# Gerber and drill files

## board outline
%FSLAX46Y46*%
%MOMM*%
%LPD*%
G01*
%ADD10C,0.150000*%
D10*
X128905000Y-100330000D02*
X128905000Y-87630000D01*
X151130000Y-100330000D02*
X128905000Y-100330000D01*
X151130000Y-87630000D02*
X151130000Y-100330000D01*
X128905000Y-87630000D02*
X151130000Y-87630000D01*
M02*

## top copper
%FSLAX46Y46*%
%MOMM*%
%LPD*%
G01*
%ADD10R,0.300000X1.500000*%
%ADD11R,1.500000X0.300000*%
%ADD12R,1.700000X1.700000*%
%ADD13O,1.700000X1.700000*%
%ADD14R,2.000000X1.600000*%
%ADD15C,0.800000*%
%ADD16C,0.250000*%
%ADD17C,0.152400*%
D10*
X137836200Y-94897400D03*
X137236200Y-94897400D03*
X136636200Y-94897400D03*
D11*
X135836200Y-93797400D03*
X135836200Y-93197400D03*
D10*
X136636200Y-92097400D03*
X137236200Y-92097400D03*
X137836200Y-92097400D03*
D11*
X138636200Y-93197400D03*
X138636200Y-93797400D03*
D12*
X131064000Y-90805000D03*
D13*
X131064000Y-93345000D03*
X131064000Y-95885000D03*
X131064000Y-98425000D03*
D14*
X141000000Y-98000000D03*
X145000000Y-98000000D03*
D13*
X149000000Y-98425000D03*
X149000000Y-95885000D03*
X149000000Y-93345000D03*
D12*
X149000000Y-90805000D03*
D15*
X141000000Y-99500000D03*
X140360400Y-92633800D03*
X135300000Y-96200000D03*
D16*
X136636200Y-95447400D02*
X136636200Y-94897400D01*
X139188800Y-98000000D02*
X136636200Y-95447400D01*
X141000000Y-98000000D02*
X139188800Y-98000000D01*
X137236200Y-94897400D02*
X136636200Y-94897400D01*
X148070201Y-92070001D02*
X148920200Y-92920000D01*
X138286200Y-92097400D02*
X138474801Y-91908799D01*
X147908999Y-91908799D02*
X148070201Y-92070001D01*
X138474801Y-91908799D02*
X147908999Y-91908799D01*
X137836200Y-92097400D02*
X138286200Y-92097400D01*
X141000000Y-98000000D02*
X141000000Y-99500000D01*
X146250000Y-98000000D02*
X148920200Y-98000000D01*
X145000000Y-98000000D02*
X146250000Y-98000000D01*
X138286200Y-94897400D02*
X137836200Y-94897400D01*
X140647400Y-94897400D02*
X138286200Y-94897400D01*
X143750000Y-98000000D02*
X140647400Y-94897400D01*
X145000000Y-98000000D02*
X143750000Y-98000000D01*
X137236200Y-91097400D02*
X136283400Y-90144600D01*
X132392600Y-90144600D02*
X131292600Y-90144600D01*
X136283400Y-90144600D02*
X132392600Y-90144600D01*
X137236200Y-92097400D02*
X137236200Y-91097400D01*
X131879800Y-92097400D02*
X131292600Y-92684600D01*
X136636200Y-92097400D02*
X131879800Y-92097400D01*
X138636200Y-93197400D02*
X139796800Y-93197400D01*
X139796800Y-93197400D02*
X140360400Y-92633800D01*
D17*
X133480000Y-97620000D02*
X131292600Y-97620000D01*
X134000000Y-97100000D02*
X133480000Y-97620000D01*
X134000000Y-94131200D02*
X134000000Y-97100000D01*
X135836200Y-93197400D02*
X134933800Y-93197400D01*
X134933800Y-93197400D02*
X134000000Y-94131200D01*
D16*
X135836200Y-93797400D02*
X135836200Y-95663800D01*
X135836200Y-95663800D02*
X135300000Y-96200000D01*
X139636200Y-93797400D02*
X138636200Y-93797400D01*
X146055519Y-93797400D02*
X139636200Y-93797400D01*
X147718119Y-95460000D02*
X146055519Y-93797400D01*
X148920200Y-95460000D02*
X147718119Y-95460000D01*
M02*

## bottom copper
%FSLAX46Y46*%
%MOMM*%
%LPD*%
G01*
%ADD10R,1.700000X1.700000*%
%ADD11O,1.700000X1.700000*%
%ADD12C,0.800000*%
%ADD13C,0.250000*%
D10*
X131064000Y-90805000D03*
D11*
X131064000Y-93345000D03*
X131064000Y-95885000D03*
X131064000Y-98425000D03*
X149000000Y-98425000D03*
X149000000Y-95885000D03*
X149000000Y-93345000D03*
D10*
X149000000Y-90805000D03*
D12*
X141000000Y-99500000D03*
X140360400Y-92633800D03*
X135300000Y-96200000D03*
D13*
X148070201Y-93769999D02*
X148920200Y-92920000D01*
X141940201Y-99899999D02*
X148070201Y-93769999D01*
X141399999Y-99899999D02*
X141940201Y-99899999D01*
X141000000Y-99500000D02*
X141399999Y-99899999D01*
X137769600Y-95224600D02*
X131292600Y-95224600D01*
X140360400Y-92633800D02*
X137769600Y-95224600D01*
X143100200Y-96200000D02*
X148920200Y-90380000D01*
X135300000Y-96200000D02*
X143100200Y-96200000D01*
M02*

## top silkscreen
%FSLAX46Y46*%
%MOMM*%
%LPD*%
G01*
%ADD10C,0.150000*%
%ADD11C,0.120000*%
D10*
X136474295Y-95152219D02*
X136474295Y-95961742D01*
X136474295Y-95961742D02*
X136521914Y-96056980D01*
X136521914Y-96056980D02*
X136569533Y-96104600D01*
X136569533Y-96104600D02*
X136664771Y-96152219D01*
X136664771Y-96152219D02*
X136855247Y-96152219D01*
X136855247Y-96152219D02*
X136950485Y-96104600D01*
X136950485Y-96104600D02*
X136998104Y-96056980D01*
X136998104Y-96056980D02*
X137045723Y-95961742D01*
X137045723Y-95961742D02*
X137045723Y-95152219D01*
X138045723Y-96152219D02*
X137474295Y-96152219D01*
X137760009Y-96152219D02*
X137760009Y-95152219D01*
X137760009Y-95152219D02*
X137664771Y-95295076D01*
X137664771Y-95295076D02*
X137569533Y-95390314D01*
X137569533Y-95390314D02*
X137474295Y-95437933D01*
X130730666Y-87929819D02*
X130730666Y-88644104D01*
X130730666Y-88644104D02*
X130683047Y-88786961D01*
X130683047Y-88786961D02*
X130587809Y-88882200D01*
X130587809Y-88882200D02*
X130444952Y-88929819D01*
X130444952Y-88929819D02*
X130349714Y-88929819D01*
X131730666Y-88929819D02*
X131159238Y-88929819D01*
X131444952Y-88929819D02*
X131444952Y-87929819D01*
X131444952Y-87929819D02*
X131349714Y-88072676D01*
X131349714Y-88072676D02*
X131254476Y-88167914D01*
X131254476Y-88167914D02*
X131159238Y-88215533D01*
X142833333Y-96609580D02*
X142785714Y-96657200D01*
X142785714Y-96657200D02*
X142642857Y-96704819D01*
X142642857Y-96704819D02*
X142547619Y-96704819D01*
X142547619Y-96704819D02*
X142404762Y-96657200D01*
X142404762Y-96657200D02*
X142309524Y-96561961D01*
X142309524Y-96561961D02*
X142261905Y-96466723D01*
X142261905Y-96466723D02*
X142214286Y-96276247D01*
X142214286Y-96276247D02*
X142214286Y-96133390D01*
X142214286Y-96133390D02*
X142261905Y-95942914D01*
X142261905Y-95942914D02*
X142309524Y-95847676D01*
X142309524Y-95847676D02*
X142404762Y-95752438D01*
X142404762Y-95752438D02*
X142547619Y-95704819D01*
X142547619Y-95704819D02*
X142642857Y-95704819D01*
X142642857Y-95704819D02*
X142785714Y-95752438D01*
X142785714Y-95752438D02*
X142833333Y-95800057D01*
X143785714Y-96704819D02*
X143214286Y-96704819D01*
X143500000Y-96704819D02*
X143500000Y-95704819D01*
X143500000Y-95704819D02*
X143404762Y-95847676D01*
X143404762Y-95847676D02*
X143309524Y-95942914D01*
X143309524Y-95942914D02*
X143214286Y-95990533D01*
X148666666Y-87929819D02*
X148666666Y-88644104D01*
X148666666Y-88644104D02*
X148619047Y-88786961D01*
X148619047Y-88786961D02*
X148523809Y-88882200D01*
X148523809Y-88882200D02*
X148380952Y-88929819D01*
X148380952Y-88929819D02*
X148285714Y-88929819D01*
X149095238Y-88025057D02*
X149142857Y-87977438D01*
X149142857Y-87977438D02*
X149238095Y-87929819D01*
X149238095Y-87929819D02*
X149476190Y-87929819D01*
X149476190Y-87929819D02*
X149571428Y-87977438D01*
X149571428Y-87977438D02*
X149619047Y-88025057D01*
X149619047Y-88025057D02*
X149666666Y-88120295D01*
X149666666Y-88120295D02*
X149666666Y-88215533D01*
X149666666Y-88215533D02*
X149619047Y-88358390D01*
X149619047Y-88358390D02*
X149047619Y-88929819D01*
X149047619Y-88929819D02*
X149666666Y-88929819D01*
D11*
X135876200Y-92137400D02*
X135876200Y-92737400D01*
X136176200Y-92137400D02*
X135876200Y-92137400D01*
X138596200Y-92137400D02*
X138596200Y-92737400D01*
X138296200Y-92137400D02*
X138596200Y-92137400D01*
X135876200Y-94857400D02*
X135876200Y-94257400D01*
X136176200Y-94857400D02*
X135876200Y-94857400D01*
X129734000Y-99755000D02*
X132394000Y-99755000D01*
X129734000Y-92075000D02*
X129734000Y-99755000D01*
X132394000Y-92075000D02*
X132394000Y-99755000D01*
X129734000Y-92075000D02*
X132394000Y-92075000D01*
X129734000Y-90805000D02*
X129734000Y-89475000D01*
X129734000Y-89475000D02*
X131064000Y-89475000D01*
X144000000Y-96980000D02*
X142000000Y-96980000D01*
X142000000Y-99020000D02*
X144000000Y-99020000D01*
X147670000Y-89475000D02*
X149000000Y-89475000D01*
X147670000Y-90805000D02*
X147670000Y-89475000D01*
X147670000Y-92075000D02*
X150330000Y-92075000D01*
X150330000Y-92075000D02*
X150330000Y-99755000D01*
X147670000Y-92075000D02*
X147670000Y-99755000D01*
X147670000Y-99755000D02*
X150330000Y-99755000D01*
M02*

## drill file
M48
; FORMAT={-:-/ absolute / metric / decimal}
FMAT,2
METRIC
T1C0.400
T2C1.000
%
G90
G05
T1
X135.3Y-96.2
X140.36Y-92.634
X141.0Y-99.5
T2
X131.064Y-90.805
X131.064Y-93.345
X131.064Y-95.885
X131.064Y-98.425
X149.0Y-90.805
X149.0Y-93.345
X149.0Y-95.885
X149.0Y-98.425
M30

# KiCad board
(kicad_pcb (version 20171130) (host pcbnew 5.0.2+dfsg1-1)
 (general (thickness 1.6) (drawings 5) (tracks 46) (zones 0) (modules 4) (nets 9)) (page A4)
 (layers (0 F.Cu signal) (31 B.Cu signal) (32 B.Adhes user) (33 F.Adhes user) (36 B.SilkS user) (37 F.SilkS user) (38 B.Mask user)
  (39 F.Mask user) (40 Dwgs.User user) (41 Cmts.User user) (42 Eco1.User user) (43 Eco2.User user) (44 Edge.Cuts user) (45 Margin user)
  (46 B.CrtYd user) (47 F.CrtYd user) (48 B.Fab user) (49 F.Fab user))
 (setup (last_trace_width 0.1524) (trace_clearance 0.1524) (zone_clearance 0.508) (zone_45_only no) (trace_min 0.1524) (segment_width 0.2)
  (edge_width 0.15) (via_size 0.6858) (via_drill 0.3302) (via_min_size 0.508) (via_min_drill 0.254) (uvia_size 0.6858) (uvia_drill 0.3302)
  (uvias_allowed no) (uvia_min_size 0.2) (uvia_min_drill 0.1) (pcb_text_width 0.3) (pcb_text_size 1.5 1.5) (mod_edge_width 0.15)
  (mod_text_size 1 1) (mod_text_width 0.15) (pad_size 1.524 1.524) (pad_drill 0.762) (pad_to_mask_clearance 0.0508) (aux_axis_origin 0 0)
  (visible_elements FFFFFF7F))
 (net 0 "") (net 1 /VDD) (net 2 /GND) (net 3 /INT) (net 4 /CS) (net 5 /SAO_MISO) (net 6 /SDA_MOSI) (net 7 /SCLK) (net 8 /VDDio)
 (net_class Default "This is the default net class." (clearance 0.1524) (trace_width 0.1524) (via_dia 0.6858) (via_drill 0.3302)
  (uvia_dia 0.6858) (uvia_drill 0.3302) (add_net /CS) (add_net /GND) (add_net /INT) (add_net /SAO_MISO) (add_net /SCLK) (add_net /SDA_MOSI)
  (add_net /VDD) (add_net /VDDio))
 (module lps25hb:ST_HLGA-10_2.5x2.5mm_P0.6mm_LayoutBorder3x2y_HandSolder (layer F.Cu) (at 137.2362 93.4974 180)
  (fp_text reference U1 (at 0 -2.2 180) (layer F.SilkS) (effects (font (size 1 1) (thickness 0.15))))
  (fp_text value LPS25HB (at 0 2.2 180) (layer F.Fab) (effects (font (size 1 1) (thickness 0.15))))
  (fp_line (start 1.36 1.36) (end 1.36 0.76) (layer F.SilkS) (width 0.12))
  (fp_line (start 1.06 1.36) (end 1.36 1.36) (layer F.SilkS) (width 0.12))
  (fp_line (start -1.36 1.36) (end -1.36 0.76) (layer F.SilkS) (width 0.12))
  (fp_line (start -1.06 1.36) (end -1.36 1.36) (layer F.SilkS) (width 0.12))
  (fp_line (start 1.36 -1.36) (end 1.36 -0.76) (layer F.SilkS) (width 0.12))
  (fp_line (start 1.06 -1.36) (end 1.36 -1.36) (layer F.SilkS) (width 0.12))
  (pad 10 smd rect (at -0.6 -1.4 180) (size 0.3 1.5) (layers F.Cu F.Paste F.Mask) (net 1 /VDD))
  (pad 9 smd rect (at 0 -1.4 180) (size 0.3 1.5) (layers F.Cu F.Paste F.Mask) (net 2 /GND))
  (pad 8 smd rect (at 0.6 -1.4 180) (size 0.3 1.5) (layers F.Cu F.Paste F.Mask) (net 2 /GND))
  (pad 7 smd rect (at 1.4 -0.3 180) (size 1.5 0.3) (layers F.Cu F.Paste F.Mask) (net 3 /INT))
  (pad 6 smd rect (at 1.4 0.3 180) (size 1.5 0.3) (layers F.Cu F.Paste F.Mask) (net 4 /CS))
  (pad 5 smd rect (at 0.6 1.4 180) (size 0.3 1.5) (layers F.Cu F.Paste F.Mask) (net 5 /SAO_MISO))
  (pad 4 smd rect (at 0 1.4 180) (size 0.3 1.5) (layers F.Cu F.Paste F.Mask) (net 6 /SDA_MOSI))
  (pad 3 smd rect (at -0.6 1.4 180) (size 0.3 1.5) (layers F.Cu F.Paste F.Mask) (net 2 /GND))
  (pad 2 smd rect (at -1.4 0.3 180) (size 1.5 0.3) (layers F.Cu F.Paste F.Mask) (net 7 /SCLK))
  (pad 1 smd rect (at -1.4 -0.3 180) (size 1.5 0.3) (layers F.Cu F.Paste F.Mask) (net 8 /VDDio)))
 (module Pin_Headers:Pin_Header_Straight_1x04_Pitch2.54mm (layer F.Cu) (at 131.064 90.805)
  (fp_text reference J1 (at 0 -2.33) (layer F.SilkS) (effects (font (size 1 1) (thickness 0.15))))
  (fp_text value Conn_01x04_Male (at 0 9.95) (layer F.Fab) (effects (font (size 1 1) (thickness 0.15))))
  (fp_line (start -1.33 8.95) (end 1.33 8.95) (layer F.SilkS) (width 0.12))
  (fp_line (start -1.33 1.27) (end -1.33 8.95) (layer F.SilkS) (width 0.12))
  (fp_line (start 1.33 1.27) (end 1.33 8.95) (layer F.SilkS) (width 0.12))
  (fp_line (start -1.33 1.27) (end 1.33 1.27) (layer F.SilkS) (width 0.12))
  (fp_line (start -1.33 0) (end -1.33 -1.33) (layer F.SilkS) (width 0.12))
  (fp_line (start -1.33 -1.33) (end 0 -1.33) (layer F.SilkS) (width 0.12))
  (pad 1 thru_hole rect (at 0 0) (size 1.7 1.7) (drill 1) (layers *.Cu *.Mask) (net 6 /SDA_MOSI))
  (pad 2 thru_hole oval (at 0 2.54) (size 1.7 1.7) (drill 1) (layers *.Cu *.Mask) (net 5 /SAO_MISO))
  (pad 3 thru_hole oval (at 0 5.08) (size 1.7 1.7) (drill 1) (layers *.Cu *.Mask) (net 7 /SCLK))
  (pad 4 thru_hole oval (at 0 7.62) (size 1.7 1.7) (drill 1) (layers *.Cu *.Mask) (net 4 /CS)))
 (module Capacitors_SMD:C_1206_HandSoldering (layer F.Cu) (at 143 98)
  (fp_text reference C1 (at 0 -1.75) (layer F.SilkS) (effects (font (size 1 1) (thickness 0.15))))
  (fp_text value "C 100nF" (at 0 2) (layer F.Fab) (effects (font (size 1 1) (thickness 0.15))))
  (fp_line (start 1 -1.02) (end -1 -1.02) (layer F.SilkS) (width 0.12))
  (fp_line (start -1 1.02) (end 1 1.02) (layer F.SilkS) (width 0.12))
  (pad 1 smd rect (at -2 0) (size 2 1.6) (layers F.Cu F.Paste F.Mask) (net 2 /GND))
  (pad 2 smd rect (at 2 0) (size 2 1.6) (layers F.Cu F.Paste F.Mask) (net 1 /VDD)))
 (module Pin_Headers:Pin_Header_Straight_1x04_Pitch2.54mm (layer F.Cu) (at 149 90.805)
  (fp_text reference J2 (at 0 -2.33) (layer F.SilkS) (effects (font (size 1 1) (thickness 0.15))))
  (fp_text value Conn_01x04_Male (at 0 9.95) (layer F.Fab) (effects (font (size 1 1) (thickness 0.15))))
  (fp_line (start -1.33 -1.33) (end 0 -1.33) (layer F.SilkS) (width 0.12))
  (fp_line (start -1.33 0) (end -1.33 -1.33) (layer F.SilkS) (width 0.12))
  (fp_line (start -1.33 1.27) (end 1.33 1.27) (layer F.SilkS) (width 0.12))
  (fp_line (start 1.33 1.27) (end 1.33 8.95) (layer F.SilkS) (width 0.12))
  (fp_line (start -1.33 1.27) (end -1.33 8.95) (layer F.SilkS) (width 0.12))
  (fp_line (start -1.33 8.95) (end 1.33 8.95) (layer F.SilkS) (width 0.12))
  (pad 4 thru_hole oval (at 0 7.62) (size 1.7 1.7) (drill 1) (layers *.Cu *.Mask) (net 1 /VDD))
  (pad 3 thru_hole oval (at 0 5.08) (size 1.7 1.7) (drill 1) (layers *.Cu *.Mask) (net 8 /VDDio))
  (pad 2 thru_hole oval (at 0 2.54) (size 1.7 1.7) (drill 1) (layers *.Cu *.Mask) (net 2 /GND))
  (pad 1 thru_hole rect (at 0 0) (size 1.7 1.7) (drill 1) (layers *.Cu *.Mask) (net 3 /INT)))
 (gr_line (start 128.905 100.33) (end 128.905 87.63) (layer Edge.Cuts) (width 0.15))
 (gr_line (start 151.13 100.33) (end 128.905 100.33) (layer Edge.Cuts) (width 0.15))
 (gr_line (start 151.13 87.63) (end 151.13 100.33) (layer Edge.Cuts) (width 0.15))
 (gr_line (start 128.905 87.63) (end 151.13 87.63) (layer Edge.Cuts) (width 0.15))
 (segment (start 136.6362 95.4474) (end 136.6362 94.8974) (width 0.25) (layer F.Cu) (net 2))
 (segment (start 139.1888 98) (end 136.6362 95.4474) (width 0.25) (layer F.Cu) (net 2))
 (segment (start 141 98) (end 139.1888 98) (width 0.25) (layer F.Cu) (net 2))
 (segment (start 137.2362 94.8974) (end 136.6362 94.8974) (width 0.25) (layer F.Cu) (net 2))
 (segment (start 148.070201 92.070001) (end 148.9202 92.92) (width 0.25) (layer F.Cu) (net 2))
 (segment (start 138.2862 92.0974) (end 138.474801 91.908799) (width 0.25) (layer F.Cu) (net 2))
 (segment (start 147.908999 91.908799) (end 148.070201 92.070001) (width 0.25) (layer F.Cu) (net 2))
 (segment (start 138.474801 91.908799) (end 147.908999 91.908799) (width 0.25) (layer F.Cu) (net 2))
 (segment (start 137.8362 92.0974) (end 138.2862 92.0974) (width 0.25) (layer F.Cu) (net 2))
 (via (at 141 99.5) (size 0.8) (drill 0.4) (layers F.Cu B.Cu) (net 2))
 (segment (start 141 98) (end 141 99.5) (width 0.25) (layer F.Cu) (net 2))
 (segment (start 148.070201 93.769999) (end 148.9202 92.92) (width 0.25) (layer B.Cu) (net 2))
 (segment (start 141.940201 99.899999) (end 148.070201 93.769999) (width 0.25) (layer B.Cu) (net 2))
 (segment (start 141.399999 99.899999) (end 141.940201 99.899999) (width 0.25) (layer B.Cu) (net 2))
 (segment (start 141 99.5) (end 141.399999 99.899999) (width 0.25) (layer B.Cu) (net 2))
 (segment (start 146.25 98) (end 148.9202 98) (width 0.25) (layer F.Cu) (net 1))
 (segment (start 145 98) (end 146.25 98) (width 0.25) (layer F.Cu) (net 1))
 (segment (start 138.2862 94.8974) (end 137.8362 94.8974) (width 0.25) (layer F.Cu) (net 1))
 (segment (start 140.6474 94.8974) (end 138.2862 94.8974) (width 0.25) (layer F.Cu) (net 1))
 (segment (start 143.75 98) (end 140.6474 94.8974) (width 0.25) (layer F.Cu) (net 1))
 (segment (start 145 98) (end 143.75 98) (width 0.25) (layer F.Cu) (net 1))
 (segment (start 137.2362 91.0974) (end 136.2834 90.1446) (width 0.25) (layer F.Cu) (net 6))
 (segment (start 132.3926 90.1446) (end 131.2926 90.1446) (width 0.25) (layer F.Cu) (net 6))
 (segment (start 136.2834 90.1446) (end 132.3926 90.1446) (width 0.25) (layer F.Cu) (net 6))
 (segment (start 137.2362 92.0974) (end 137.2362 91.0974) (width 0.25) (layer F.Cu) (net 6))
 (segment (start 131.8798 92.0974) (end 131.2926 92.6846) (width 0.25) (layer F.Cu) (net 5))
 (segment (start 136.6362 92.0974) (end 131.8798 92.0974) (width 0.25) (layer F.Cu) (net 5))
 (via (at 140.3604 92.6338) (size 0.8) (drill 0.4) (layers F.Cu B.Cu) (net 7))
 (segment (start 138.6362 93.1974) (end 139.7968 93.1974) (width 0.25) (layer F.Cu) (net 7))
 (segment (start 139.7968 93.1974) (end 140.3604 92.6338) (width 0.25) (layer F.Cu) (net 7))
 (segment (start 137.7696 95.2246) (end 131.2926 95.2246) (width 0.25) (layer B.Cu) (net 7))
 (segment (start 140.3604 92.6338) (end 137.7696 95.2246) (width 0.25) (layer B.Cu) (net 7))
 (segment (start 133.48 97.62) (end 131.2926 97.62) (width 0.1524) (layer F.Cu) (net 4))
 (segment (start 134 97.1) (end 133.48 97.62) (width 0.1524) (layer F.Cu) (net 4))
 (segment (start 134 94.1312) (end 134 97.1) (width 0.1524) (layer F.Cu) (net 4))
 (segment (start 135.8362 93.1974) (end 134.9338 93.1974) (width 0.1524) (layer F.Cu) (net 4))
 (segment (start 134.9338 93.1974) (end 134 94.1312) (width 0.1524) (layer F.Cu) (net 4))
 (via (at 135.3 96.2) (size 0.8) (drill 0.4) (layers F.Cu B.Cu) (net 3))
 (segment (start 135.8362 93.7974) (end 135.8362 95.6638) (width 0.25) (layer F.Cu) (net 3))
 (segment (start 135.8362 95.6638) (end 135.3 96.2) (width 0.25) (layer F.Cu) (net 3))
 (segment (start 143.1002 96.2) (end 148.9202 90.38) (width 0.25) (layer B.Cu) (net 3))
 (segment (start 135.3 96.2) (end 143.1002 96.2) (width 0.25) (layer B.Cu) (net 3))
 (segment (start 139.6362 93.7974) (end 138.6362 93.7974) (width 0.25) (layer F.Cu) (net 8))
 (segment (start 146.055519 93.7974) (end 139.6362 93.7974) (width 0.25) (layer F.Cu) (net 8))
 (segment (start 147.718119 95.46) (end 146.055519 93.7974) (width 0.25) (layer F.Cu) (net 8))
 (segment (start 148.9202 95.46) (end 147.718119 95.46) (width 0.25) (layer F.Cu) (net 8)))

